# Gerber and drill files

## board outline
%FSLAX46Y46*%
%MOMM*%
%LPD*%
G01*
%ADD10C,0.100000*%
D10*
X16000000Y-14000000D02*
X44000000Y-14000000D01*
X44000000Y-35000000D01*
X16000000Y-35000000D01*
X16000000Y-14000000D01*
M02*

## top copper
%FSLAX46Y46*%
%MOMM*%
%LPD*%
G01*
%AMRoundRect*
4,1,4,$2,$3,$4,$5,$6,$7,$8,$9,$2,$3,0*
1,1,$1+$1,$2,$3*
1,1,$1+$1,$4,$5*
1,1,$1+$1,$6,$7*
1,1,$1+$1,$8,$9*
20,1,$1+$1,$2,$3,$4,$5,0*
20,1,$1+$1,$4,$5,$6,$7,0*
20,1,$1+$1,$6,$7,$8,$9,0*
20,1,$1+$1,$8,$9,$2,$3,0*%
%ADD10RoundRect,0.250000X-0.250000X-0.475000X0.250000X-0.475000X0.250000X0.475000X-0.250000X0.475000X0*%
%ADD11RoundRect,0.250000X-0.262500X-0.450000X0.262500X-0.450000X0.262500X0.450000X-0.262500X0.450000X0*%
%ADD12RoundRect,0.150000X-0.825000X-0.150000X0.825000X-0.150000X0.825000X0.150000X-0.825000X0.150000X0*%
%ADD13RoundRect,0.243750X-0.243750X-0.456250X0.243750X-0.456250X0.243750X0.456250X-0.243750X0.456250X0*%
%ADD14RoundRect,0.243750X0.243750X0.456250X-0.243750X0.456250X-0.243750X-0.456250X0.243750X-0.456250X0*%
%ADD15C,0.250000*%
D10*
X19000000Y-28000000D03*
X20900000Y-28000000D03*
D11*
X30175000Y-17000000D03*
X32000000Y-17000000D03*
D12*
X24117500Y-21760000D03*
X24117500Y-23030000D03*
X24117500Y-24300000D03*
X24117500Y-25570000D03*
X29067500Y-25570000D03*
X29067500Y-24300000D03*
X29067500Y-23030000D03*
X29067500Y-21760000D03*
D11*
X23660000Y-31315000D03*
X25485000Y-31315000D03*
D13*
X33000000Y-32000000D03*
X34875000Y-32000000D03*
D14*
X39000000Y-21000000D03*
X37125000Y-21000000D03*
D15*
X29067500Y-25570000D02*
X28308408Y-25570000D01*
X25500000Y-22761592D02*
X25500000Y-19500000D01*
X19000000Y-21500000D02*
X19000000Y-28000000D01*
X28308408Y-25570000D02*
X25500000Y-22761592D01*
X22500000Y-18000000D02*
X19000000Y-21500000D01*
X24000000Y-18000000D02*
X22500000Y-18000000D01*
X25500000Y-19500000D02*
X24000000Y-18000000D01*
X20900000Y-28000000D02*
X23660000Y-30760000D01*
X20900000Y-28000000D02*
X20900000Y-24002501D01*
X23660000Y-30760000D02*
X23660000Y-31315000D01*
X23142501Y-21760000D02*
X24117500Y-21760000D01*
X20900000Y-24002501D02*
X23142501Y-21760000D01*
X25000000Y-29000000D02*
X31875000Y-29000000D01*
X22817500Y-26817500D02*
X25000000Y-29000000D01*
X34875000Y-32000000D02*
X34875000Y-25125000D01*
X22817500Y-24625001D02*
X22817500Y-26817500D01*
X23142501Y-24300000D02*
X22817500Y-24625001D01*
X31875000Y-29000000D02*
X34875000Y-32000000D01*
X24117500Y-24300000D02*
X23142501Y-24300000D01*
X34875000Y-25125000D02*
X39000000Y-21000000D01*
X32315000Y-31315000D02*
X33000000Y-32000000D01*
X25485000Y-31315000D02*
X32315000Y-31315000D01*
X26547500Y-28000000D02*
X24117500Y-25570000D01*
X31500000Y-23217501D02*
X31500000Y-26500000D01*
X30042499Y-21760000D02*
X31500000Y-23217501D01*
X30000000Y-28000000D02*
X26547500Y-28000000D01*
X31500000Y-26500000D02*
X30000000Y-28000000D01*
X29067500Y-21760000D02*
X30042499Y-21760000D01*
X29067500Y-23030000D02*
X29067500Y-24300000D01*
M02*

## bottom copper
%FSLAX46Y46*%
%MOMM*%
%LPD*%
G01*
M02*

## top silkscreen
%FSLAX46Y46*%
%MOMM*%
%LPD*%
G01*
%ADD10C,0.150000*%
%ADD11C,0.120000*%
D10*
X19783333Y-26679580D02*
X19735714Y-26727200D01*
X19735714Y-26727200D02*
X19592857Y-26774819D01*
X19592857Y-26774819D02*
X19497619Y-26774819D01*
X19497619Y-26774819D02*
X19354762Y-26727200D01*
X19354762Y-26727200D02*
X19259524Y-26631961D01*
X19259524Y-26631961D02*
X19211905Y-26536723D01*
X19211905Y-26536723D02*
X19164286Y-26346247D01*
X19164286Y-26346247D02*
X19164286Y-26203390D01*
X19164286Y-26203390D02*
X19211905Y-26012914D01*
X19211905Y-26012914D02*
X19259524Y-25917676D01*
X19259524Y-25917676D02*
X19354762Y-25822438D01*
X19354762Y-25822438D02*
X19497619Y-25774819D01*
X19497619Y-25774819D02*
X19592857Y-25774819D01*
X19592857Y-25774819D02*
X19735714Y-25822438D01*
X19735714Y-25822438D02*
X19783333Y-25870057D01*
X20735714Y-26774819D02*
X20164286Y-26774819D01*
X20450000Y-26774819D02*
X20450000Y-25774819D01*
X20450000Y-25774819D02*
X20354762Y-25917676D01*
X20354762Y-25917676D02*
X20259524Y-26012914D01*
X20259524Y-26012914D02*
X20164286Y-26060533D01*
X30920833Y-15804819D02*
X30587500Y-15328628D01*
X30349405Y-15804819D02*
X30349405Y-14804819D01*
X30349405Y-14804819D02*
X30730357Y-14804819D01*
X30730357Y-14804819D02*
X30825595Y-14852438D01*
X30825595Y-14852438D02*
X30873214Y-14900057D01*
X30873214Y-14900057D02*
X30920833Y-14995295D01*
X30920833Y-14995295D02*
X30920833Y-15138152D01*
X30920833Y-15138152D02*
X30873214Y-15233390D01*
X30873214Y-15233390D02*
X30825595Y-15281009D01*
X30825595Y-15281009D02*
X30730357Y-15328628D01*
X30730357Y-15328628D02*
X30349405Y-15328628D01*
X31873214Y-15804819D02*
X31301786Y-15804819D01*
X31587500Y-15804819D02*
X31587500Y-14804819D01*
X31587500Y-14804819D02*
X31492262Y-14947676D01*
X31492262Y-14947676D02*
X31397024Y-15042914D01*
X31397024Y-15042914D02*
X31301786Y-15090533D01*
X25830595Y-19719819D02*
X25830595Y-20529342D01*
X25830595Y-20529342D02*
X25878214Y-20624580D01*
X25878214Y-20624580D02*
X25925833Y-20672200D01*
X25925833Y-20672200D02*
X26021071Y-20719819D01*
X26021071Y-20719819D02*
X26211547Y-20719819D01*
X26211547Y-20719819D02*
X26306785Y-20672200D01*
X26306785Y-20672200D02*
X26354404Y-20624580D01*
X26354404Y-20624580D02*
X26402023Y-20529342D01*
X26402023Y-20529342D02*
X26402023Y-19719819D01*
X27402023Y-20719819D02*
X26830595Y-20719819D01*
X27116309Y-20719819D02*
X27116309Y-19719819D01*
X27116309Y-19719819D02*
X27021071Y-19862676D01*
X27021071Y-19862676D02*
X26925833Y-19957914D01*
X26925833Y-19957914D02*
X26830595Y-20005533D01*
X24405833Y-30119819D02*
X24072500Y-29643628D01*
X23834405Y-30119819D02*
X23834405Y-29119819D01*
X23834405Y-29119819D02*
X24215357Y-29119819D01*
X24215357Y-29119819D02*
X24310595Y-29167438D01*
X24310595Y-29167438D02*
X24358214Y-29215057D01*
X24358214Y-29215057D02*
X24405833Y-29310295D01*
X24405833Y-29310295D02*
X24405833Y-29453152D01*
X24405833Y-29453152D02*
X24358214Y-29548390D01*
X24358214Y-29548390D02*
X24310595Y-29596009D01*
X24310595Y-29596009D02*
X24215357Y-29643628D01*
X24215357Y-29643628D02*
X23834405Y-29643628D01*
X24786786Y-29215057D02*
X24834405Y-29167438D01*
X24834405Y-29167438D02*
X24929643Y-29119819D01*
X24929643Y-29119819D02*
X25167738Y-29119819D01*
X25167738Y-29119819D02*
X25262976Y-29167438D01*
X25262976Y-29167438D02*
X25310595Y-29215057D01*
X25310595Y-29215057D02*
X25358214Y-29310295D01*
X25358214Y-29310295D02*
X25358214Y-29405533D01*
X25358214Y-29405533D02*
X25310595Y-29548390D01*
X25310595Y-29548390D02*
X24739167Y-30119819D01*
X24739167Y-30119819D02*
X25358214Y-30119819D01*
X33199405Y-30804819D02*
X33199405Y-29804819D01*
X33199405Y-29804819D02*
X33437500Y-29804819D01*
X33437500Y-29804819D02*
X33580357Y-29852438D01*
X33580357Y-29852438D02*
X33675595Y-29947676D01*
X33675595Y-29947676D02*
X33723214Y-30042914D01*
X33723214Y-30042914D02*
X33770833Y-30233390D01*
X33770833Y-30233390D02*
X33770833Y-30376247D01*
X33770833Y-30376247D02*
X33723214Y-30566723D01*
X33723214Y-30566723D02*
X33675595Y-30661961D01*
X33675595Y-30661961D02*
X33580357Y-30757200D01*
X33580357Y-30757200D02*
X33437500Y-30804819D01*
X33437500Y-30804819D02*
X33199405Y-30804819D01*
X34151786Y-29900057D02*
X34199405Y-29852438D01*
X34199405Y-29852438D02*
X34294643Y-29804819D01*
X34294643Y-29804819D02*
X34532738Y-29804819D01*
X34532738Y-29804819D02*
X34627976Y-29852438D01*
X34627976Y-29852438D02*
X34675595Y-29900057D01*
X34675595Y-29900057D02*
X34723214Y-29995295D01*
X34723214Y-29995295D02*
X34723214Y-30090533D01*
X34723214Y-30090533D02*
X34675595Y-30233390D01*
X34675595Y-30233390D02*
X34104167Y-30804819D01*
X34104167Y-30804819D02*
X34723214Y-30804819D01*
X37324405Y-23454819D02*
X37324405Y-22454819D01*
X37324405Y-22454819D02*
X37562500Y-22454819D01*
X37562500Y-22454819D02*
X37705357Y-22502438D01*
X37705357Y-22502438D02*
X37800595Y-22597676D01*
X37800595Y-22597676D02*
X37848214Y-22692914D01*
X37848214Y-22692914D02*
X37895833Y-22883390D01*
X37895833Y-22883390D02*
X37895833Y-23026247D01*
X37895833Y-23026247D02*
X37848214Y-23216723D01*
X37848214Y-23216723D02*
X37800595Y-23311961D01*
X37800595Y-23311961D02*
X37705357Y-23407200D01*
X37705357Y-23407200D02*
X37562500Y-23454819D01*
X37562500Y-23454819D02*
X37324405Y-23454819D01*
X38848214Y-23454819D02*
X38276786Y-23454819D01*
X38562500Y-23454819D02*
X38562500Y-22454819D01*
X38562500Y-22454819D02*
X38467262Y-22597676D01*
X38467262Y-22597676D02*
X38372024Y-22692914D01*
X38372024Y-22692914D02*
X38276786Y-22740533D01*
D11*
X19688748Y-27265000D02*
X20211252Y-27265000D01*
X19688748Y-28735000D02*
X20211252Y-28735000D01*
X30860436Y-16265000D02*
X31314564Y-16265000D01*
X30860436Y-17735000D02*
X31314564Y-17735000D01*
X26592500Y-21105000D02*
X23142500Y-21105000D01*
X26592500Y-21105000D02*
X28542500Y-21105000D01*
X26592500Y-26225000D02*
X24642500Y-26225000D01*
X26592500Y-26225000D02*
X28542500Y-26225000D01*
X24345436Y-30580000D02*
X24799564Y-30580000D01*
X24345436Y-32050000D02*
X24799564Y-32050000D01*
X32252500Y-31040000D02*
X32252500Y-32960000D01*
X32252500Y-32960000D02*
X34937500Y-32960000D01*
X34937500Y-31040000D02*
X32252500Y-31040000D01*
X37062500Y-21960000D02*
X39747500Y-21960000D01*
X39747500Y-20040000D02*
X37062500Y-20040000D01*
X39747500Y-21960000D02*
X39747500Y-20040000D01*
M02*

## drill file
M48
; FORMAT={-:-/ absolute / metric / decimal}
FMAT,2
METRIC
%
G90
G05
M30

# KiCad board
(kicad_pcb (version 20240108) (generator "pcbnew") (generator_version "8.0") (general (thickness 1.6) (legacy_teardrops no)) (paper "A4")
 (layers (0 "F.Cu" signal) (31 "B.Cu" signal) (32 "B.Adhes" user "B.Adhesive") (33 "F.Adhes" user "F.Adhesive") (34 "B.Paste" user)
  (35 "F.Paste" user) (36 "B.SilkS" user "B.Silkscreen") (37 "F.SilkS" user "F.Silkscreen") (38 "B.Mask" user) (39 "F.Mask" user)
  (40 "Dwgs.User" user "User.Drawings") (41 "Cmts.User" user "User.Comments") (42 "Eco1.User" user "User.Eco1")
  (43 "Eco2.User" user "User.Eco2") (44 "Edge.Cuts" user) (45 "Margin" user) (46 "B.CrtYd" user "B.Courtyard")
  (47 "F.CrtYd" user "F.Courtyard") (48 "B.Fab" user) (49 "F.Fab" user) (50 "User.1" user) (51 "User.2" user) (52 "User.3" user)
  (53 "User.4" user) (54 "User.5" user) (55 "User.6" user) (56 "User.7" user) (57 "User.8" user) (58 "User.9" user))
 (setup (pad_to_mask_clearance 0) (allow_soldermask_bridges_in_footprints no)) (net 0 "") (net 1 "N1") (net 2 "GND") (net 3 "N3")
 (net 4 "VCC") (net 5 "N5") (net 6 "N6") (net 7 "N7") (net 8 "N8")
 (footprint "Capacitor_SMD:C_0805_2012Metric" (layer "F.Cu") (at 19.95 28)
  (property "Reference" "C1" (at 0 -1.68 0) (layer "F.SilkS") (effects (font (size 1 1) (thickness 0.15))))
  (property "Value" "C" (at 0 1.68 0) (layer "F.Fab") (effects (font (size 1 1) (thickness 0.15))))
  (fp_line (start -0.261252 -0.735) (end 0.261252 -0.735) (stroke (width 0.12) (type solid)) (layer "F.SilkS"))
  (fp_line (start -0.261252 0.735) (end 0.261252 0.735) (stroke (width 0.12) (type solid)) (layer "F.SilkS"))
  (pad "1" smd roundrect (at -0.95 0) (size 1 1.45) (layers "F.Cu" "F.Paste" "F.Mask") (roundrect_rratio 0.25) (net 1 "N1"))
  (pad "2" smd roundrect (at 0.95 0) (size 1 1.45) (layers "F.Cu" "F.Paste" "F.Mask") (roundrect_rratio 0.25) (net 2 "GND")))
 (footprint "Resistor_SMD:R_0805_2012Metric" (layer "F.Cu") (at 31.0875 17)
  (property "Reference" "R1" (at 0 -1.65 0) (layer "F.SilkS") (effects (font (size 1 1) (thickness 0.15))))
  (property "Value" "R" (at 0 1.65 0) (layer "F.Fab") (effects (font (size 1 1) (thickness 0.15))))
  (fp_line (start -0.227064 -0.735) (end 0.227064 -0.735) (stroke (width 0.12) (type solid)) (layer "F.SilkS"))
  (fp_line (start -0.227064 0.735) (end 0.227064 0.735) (stroke (width 0.12) (type solid)) (layer "F.SilkS"))
  (pad "1" smd roundrect (at -0.9125 0) (size 1.025 1.4) (layers "F.Cu" "F.Paste" "F.Mask") (roundrect_rratio 0.243902) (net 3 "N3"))
  (pad "2" smd roundrect (at 0.9125 0) (size 1.025 1.4) (layers "F.Cu" "F.Paste" "F.Mask") (roundrect_rratio 0.243902) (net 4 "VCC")))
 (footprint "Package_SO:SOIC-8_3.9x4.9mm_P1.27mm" (layer "F.Cu") (at 26.5925 23.665)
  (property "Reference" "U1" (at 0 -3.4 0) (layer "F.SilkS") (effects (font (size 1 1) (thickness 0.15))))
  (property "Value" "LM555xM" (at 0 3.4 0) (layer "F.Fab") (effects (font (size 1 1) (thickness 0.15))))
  (fp_line (start 0 -2.56) (end -3.45 -2.56) (stroke (width 0.12) (type solid)) (layer "F.SilkS"))
  (fp_line (start 0 -2.56) (end 1.95 -2.56) (stroke (width 0.12) (type solid)) (layer "F.SilkS"))
  (fp_line (start 0 2.56) (end -1.95 2.56) (stroke (width 0.12) (type solid)) (layer "F.SilkS"))
  (fp_line (start 0 2.56) (end 1.95 2.56) (stroke (width 0.12) (type solid)) (layer "F.SilkS"))
  (pad "1" smd roundrect (at -2.475 -1.905) (size 1.95 0.6) (layers "F.Cu" "F.Paste" "F.Mask") (roundrect_rratio 0.25) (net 2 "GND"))
  (pad "2" smd roundrect (at -2.475 -0.635) (size 1.95 0.6) (layers "F.Cu" "F.Paste" "F.Mask") (roundrect_rratio 0.25) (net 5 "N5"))
  (pad "3" smd roundrect (at -2.475 0.635) (size 1.95 0.6) (layers "F.Cu" "F.Paste" "F.Mask") (roundrect_rratio 0.25) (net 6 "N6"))
  (pad "4" smd roundrect (at -2.475 1.905) (size 1.95 0.6) (layers "F.Cu" "F.Paste" "F.Mask") (roundrect_rratio 0.25) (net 4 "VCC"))
  (pad "5" smd roundrect (at 2.475 1.905) (size 1.95 0.6) (layers "F.Cu" "F.Paste" "F.Mask") (roundrect_rratio 0.25) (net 1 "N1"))
  (pad "6" smd roundrect (at 2.475 0.635) (size 1.95 0.6) (layers "F.Cu" "F.Paste" "F.Mask") (roundrect_rratio 0.25) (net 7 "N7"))
  (pad "7" smd roundrect (at 2.475 -0.635) (size 1.95 0.6) (layers "F.Cu" "F.Paste" "F.Mask") (roundrect_rratio 0.25) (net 7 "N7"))
  (pad "8" smd roundrect (at 2.475 -1.905) (size 1.95 0.6) (layers "F.Cu" "F.Paste" "F.Mask") (roundrect_rratio 0.25) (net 4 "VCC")))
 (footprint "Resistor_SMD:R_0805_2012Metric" (layer "F.Cu") (at 24.5725 31.315)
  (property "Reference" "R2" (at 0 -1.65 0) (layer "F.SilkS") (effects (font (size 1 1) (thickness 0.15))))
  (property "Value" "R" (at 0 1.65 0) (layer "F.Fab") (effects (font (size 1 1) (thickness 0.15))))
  (fp_line (start -0.227064 -0.735) (end 0.227064 -0.735) (stroke (width 0.12) (type solid)) (layer "F.SilkS"))
  (fp_line (start -0.227064 0.735) (end 0.227064 0.735) (stroke (width 0.12) (type solid)) (layer "F.SilkS"))
  (pad "1" smd roundrect (at -0.9125 0) (size 1.025 1.4) (layers "F.Cu" "F.Paste" "F.Mask") (roundrect_rratio 0.243902) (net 2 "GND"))
  (pad "2" smd roundrect (at 0.9125 0) (size 1.025 1.4) (layers "F.Cu" "F.Paste" "F.Mask") (roundrect_rratio 0.243902) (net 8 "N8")))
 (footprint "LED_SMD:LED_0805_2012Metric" (layer "F.Cu") (at 33.9375 32)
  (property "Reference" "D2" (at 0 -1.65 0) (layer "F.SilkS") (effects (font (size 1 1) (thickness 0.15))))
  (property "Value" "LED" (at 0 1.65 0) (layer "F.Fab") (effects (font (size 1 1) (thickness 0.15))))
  (fp_line (start -1.685 -0.96) (end -1.685 0.96) (stroke (width 0.12) (type solid)) (layer "F.SilkS"))
  (fp_line (start -1.685 0.96) (end 1 0.96) (stroke (width 0.12) (type solid)) (layer "F.SilkS"))
  (fp_line (start 1 -0.96) (end -1.685 -0.96) (stroke (width 0.12) (type solid)) (layer "F.SilkS"))
  (pad "1" smd roundrect (at -0.9375 0) (size 0.975 1.4) (layers "F.Cu" "F.Paste" "F.Mask") (roundrect_rratio 0.25) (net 8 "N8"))
  (pad "2" smd roundrect (at 0.9375 0) (size 0.975 1.4) (layers "F.Cu" "F.Paste" "F.Mask") (roundrect_rratio 0.25) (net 6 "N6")))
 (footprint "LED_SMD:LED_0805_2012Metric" (layer "F.Cu") (at 38.0625 21 180)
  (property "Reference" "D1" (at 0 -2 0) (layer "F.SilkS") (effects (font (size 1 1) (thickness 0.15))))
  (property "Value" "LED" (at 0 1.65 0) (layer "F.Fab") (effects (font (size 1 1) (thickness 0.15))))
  (fp_line (start 1 -0.96) (end -1.685 -0.96) (stroke (width 0.12) (type solid)) (layer "F.SilkS"))
  (fp_line (start -1.685 0.96) (end 1 0.96) (stroke (width 0.12) (type solid)) (layer "F.SilkS"))
  (fp_line (start -1.685 -0.96) (end -1.685 0.96) (stroke (width 0.12) (type solid)) (layer "F.SilkS"))
  (pad "1" smd roundrect (at -0.9375 0 180) (size 0.975 1.4) (layers "F.Cu" "F.Paste" "F.Mask") (roundrect_rratio 0.25) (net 6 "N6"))
  (pad "2" smd roundrect (at 0.9375 0 180) (size 0.975 1.4) (layers "F.Cu" "F.Paste" "F.Mask") (roundrect_rratio 0.25) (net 3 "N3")))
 (gr_rect (start 16 14) (end 44 35) (stroke (width 0.1) (type default)) (fill none) (layer "Edge.Cuts"))
 (segment (start 29.0675 25.57) (end 28.308408 25.57) (width 0.25) (layer "F.Cu") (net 1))
 (segment (start 25.5 22.761592) (end 25.5 19.5) (width 0.25) (layer "F.Cu") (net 1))
 (segment (start 19 21.5) (end 19 28) (width 0.25) (layer "F.Cu") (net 1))
 (segment (start 28.308408 25.57) (end 25.5 22.761592) (width 0.25) (layer "F.Cu") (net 1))
 (segment (start 22.5 18) (end 19 21.5) (width 0.25) (layer "F.Cu") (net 1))
 (segment (start 24 18) (end 22.5 18) (width 0.25) (layer "F.Cu") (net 1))
 (segment (start 25.5 19.5) (end 24 18) (width 0.25) (layer "F.Cu") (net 1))
 (segment (start 20.9 28) (end 23.66 30.76) (width 0.25) (layer "F.Cu") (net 2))
 (segment (start 20.9 28) (end 20.9 24.002501) (width 0.25) (layer "F.Cu") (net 2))
 (segment (start 23.66 30.76) (end 23.66 31.315) (width 0.25) (layer "F.Cu") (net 2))
 (segment (start 23.142501 21.76) (end 24.1175 21.76) (width 0.25) (layer "F.Cu") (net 2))
 (segment (start 20.9 24.002501) (end 23.142501 21.76) (width 0.25) (layer "F.Cu") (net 2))
 (segment (start 25 29) (end 31.875 29) (width 0.25) (layer "F.Cu") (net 6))
 (segment (start 22.8175 26.8175) (end 25 29) (width 0.25) (layer "F.Cu") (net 6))
 (segment (start 34.875 32) (end 34.875 25.125) (width 0.25) (layer "F.Cu") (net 6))
 (segment (start 22.8175 24.625001) (end 22.8175 26.8175) (width 0.25) (layer "F.Cu") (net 6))
 (segment (start 23.142501 24.3) (end 22.8175 24.625001) (width 0.25) (layer "F.Cu") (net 6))
 (segment (start 31.875 29) (end 34.875 32) (width 0.25) (layer "F.Cu") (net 6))
 (segment (start 24.1175 24.3) (end 23.142501 24.3) (width 0.25) (layer "F.Cu") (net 6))
 (segment (start 34.875 25.125) (end 39 21) (width 0.25) (layer "F.Cu") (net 6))
 (segment (start 32.315 31.315) (end 33 32) (width 0.25) (layer "F.Cu") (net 8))
 (segment (start 25.485 31.315) (end 32.315 31.315) (width 0.25) (layer "F.Cu") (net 8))
 (segment (start 26.5475 28) (end 24.1175 25.57) (width 0.25) (layer "F.Cu") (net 4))
 (segment (start 31.5 23.217501) (end 31.5 26.5) (width 0.25) (layer "F.Cu") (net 4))
 (segment (start 30.042499 21.76) (end 31.5 23.217501) (width 0.25) (layer "F.Cu") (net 4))
 (segment (start 30 28) (end 26.5475 28) (width 0.25) (layer "F.Cu") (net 4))
 (segment (start 31.5 26.5) (end 30 28) (width 0.25) (layer "F.Cu") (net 4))
 (segment (start 29.0675 21.76) (end 30.042499 21.76) (width 0.25) (layer "F.Cu") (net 4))
 (segment (start 29.0675 23.03) (end 29.0675 24.3) (width 0.25) (layer "F.Cu") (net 7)))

